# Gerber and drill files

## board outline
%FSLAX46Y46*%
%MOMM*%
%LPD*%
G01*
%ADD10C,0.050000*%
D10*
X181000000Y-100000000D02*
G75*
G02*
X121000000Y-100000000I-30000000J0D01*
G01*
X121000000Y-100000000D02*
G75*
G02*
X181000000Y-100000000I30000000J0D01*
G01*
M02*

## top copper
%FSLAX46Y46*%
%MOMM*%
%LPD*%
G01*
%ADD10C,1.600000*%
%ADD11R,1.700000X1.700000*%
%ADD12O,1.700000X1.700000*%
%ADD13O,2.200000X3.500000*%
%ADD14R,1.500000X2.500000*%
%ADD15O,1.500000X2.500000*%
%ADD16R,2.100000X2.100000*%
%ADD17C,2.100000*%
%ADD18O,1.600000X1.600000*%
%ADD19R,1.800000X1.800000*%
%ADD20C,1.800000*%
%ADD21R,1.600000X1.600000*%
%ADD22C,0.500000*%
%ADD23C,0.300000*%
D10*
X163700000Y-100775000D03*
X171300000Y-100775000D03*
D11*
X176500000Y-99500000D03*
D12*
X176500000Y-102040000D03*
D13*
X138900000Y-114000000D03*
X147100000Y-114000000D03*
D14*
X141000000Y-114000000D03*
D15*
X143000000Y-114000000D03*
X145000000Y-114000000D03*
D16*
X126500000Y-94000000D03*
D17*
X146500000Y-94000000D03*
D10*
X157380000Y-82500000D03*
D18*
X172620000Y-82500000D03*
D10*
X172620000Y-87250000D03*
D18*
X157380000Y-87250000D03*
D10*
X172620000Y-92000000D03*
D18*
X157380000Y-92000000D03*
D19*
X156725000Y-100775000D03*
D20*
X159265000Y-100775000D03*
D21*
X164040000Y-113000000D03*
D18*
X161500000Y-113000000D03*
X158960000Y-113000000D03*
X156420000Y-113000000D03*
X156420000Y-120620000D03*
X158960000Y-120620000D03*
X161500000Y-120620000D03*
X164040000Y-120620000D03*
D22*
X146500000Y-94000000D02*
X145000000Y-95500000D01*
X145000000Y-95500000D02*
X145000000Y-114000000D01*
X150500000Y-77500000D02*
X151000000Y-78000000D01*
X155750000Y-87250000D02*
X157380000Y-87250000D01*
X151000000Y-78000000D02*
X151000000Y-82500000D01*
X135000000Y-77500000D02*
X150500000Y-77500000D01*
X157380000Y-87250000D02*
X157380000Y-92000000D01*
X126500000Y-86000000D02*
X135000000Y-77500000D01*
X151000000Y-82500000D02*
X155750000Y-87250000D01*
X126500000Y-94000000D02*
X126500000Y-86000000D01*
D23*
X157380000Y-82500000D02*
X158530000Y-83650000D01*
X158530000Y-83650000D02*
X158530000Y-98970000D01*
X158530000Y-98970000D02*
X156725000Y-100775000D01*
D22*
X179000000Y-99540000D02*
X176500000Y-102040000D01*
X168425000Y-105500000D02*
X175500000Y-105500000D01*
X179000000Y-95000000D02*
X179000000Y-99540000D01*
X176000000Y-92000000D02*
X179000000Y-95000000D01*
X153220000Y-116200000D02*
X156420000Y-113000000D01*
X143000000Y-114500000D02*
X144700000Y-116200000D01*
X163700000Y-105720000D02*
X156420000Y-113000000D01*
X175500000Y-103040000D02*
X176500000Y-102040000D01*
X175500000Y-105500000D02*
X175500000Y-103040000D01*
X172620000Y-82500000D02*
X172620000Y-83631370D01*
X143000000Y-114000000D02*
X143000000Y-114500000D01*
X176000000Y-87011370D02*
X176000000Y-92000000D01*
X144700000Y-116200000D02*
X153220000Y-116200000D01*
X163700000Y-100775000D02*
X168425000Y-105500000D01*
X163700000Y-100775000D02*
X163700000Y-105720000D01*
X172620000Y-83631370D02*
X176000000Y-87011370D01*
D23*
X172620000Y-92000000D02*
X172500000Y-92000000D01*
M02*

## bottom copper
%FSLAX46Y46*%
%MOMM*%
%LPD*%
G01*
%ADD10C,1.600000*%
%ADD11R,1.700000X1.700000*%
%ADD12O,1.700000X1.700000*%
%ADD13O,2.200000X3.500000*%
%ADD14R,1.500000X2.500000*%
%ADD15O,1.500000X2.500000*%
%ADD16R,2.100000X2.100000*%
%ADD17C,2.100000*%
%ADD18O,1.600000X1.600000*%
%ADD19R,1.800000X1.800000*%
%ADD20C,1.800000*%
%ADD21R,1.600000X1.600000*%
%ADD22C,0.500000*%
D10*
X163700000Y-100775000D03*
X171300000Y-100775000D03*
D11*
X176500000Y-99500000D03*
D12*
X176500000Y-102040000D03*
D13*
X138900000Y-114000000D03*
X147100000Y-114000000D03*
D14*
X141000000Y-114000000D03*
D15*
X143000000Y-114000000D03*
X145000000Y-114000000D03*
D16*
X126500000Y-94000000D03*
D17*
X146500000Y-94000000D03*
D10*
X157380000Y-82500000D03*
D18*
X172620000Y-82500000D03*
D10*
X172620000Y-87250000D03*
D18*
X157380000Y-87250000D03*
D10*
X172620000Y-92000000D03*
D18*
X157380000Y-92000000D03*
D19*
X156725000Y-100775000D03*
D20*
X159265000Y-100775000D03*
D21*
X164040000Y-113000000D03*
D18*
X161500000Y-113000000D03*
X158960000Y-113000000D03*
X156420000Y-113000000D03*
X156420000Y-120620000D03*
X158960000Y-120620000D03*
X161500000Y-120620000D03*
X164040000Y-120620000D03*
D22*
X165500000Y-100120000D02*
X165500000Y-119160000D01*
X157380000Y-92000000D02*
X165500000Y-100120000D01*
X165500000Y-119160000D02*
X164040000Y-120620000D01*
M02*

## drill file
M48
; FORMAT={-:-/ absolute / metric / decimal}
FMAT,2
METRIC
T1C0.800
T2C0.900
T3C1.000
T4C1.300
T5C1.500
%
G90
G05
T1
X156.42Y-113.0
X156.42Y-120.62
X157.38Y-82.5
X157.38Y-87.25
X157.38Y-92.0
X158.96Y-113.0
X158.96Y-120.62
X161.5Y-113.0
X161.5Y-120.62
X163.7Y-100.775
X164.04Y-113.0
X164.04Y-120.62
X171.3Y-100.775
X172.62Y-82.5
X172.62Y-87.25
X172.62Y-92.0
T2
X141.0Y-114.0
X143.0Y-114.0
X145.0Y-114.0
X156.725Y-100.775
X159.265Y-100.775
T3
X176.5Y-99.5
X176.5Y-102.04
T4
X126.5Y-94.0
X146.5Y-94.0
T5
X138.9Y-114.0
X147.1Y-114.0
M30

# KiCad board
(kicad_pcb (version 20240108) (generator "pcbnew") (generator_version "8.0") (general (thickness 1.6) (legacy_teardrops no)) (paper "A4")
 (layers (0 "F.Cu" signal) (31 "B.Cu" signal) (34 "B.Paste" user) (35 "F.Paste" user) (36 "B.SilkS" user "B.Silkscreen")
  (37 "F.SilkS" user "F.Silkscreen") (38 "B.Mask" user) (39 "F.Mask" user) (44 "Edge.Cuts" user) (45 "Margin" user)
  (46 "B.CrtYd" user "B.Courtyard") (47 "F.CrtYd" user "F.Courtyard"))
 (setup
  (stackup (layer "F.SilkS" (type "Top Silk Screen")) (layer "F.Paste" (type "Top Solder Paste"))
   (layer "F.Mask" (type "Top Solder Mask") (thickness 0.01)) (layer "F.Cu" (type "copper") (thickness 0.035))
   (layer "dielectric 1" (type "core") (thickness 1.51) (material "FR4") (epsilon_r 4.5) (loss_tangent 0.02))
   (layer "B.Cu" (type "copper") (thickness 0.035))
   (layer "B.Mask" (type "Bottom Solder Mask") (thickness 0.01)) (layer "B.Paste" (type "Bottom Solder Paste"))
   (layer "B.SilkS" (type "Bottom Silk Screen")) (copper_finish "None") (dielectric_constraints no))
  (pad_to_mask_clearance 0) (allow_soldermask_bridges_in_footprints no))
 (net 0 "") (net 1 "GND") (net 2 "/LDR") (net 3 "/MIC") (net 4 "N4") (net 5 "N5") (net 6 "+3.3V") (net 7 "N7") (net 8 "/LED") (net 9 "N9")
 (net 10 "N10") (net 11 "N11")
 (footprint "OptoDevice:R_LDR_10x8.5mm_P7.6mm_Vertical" (layer "F.Cu") (at 163.7 100.775)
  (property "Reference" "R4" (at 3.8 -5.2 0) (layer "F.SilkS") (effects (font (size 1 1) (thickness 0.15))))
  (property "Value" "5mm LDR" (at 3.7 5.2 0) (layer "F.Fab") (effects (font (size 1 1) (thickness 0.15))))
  (pad "1" thru_hole circle (at 0 0) (size 1.6 1.6) (drill 0.8) (layers "*.Cu" "*.Mask") (remove_unused_layers no) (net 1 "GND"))
  (pad "2" thru_hole circle (at 7.6 0) (size 1.6 1.6) (drill 0.8) (layers "*.Cu" "*.Mask") (remove_unused_layers no) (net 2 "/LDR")))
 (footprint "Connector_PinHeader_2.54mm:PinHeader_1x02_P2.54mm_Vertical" (layer "F.Cu") (at 176.5 99.5)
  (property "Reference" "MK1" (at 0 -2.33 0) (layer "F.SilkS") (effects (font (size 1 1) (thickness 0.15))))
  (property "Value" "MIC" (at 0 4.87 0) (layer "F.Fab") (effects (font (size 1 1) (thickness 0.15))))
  (pad "1" thru_hole rect (at 0 0) (size 1.7 1.7) (drill 1) (layers "*.Cu" "*.Mask") (remove_unused_layers no) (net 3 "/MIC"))
  (pad "2" thru_hole oval (at 0 2.54) (size 1.7 1.7) (drill 1) (layers "*.Cu" "*.Mask") (remove_unused_layers no) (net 1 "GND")))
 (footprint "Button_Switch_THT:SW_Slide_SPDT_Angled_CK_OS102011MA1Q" (layer "F.Cu") (at 141 114)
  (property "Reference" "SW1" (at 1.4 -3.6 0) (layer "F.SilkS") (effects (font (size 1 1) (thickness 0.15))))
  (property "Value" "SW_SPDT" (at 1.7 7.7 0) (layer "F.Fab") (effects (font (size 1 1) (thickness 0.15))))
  (pad "" thru_hole oval (at -2.1 0) (size 2.2 3.5) (drill 1.5) (layers "*.Cu" "*.Mask") (remove_unused_layers no))
  (pad "" thru_hole oval (at 6.1 0) (size 2.2 3.5) (drill 1.5) (layers "*.Cu" "*.Mask") (remove_unused_layers no))
  (pad "1" thru_hole rect (at 0 0) (size 1.5 2.5) (drill 0.9) (layers "*.Cu" "*.Mask") (remove_unused_layers no) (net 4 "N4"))
  (pad "2" thru_hole oval (at 2 0) (size 1.5 2.5) (drill 0.9) (layers "*.Cu" "*.Mask") (remove_unused_layers no) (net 1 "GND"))
  (pad "3" thru_hole oval (at 4 0) (size 1.5 2.5) (drill 0.9) (layers "*.Cu" "*.Mask") (remove_unused_layers no) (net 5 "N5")))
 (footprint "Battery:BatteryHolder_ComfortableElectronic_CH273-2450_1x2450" (layer "F.Cu") (at 126.5 94)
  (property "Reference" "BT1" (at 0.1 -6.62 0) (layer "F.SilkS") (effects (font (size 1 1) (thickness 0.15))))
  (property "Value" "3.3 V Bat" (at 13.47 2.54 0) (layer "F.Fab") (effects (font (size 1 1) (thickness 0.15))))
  (pad "1" thru_hole rect (at 0 0 270) (size 2.1 2.1) (drill 1.3) (layers "*.Cu" "*.Mask") (remove_unused_layers no) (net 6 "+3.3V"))
  (pad "2" thru_hole circle (at 20 0 270) (size 2.1 2.1) (drill 1.3) (layers "*.Cu" "*.Mask") (remove_unused_layers no) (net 5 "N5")))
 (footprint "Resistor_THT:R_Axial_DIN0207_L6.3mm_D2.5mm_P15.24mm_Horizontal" (layer "F.Cu") (at 157.38 82.5)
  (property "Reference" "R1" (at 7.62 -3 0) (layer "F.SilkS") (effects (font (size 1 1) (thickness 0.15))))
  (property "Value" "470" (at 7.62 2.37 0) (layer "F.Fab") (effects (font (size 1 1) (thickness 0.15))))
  (pad "1" thru_hole circle (at 0 0) (size 1.6 1.6) (drill 0.8) (layers "*.Cu" "*.Mask") (remove_unused_layers no) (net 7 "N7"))
  (pad "2" thru_hole oval (at 15.24 0) (size 1.6 1.6) (drill 0.8) (layers "*.Cu" "*.Mask") (remove_unused_layers no) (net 1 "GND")))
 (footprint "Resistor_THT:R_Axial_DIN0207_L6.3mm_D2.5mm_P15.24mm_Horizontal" (layer "F.Cu") (at 172.62 87.25 180)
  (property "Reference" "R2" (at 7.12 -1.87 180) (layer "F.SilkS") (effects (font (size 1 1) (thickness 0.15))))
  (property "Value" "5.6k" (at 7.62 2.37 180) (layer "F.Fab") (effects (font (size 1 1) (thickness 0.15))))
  (pad "1" thru_hole circle (at 0 0 180) (size 1.6 1.6) (drill 0.8) (layers "*.Cu" "*.Mask") (remove_unused_layers no) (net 3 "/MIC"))
  (pad "2" thru_hole oval (at 15.24 0 180) (size 1.6 1.6) (drill 0.8) (layers "*.Cu" "*.Mask") (remove_unused_layers no) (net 6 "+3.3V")))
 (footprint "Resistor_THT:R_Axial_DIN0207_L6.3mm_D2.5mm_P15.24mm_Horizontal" (layer "F.Cu") (at 172.62 92 180)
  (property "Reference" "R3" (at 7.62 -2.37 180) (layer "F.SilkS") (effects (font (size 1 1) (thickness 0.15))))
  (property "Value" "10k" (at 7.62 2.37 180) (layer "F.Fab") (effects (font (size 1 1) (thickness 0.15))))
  (pad "1" thru_hole circle (at 0 0 180) (size 1.6 1.6) (drill 0.8) (layers "*.Cu" "*.Mask") (remove_unused_layers no) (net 2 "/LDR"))
  (pad "2" thru_hole oval (at 15.24 0 180) (size 1.6 1.6) (drill 0.8) (layers "*.Cu" "*.Mask") (remove_unused_layers no) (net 6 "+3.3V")))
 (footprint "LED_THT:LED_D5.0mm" (layer "F.Cu") (at 156.725 100.775)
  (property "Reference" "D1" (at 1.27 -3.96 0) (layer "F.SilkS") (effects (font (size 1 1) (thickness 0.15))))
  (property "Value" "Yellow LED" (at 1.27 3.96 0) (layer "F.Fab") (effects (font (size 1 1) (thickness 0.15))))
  (pad "1" thru_hole rect (at 0 0) (size 1.8 1.8) (drill 0.9) (layers "*.Cu" "*.Mask") (remove_unused_layers no) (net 7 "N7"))
  (pad "2" thru_hole circle (at 2.54 0) (size 1.8 1.8) (drill 0.9) (layers "*.Cu" "*.Mask") (remove_unused_layers no) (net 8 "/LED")))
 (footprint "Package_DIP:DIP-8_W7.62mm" (layer "F.Cu") (at 164.04 113 -90)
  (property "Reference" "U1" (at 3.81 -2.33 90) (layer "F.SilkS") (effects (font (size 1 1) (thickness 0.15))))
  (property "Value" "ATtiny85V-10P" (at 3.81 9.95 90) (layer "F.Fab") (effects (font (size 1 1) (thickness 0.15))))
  (pad "1" thru_hole rect (at 0 0 270) (size 1.6 1.6) (drill 0.8) (layers "*.Cu" "*.Mask") (remove_unused_layers no) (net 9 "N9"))
  (pad "2" thru_hole oval (at 0 2.54 270) (size 1.6 1.6) (drill 0.8) (layers "*.Cu" "*.Mask") (remove_unused_layers no) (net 3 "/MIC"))
  (pad "3" thru_hole oval (at 0 5.08 270) (size 1.6 1.6) (drill 0.8) (layers "*.Cu" "*.Mask") (remove_unused_layers no) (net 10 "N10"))
  (pad "4" thru_hole oval (at 0 7.62 270) (size 1.6 1.6) (drill 0.8) (layers "*.Cu" "*.Mask") (remove_unused_layers no) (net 1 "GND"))
  (pad "5" thru_hole oval (at 7.62 7.62 270) (size 1.6 1.6) (drill 0.8) (layers "*.Cu" "*.Mask") (remove_unused_layers no) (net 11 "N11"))
  (pad "6" thru_hole oval (at 7.62 5.08 270) (size 1.6 1.6) (drill 0.8) (layers "*.Cu" "*.Mask") (remove_unused_layers no) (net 8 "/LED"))
  (pad "7" thru_hole oval (at 7.62 2.54 270) (size 1.6 1.6) (drill 0.8) (layers "*.Cu" "*.Mask") (remove_unused_layers no) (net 2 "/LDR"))
  (pad "8" thru_hole oval (at 7.62 0 270) (size 1.6 1.6) (drill 0.8) (layers "*.Cu" "*.Mask") (remove_unused_layers no) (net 6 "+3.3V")))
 (gr_circle (center 151 100) (end 181 100) (stroke (width 0.05) (type default)) (fill none) (layer "Edge.Cuts"))
 (segment (start 146.5 94) (end 145 95.5) (width 0.5) (layer "F.Cu") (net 5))
 (segment (start 145 95.5) (end 145 114) (width 0.5) (layer "F.Cu") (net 5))
 (segment (start 150.5 77.5) (end 151 78) (width 0.5) (layer "F.Cu") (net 6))
 (segment (start 155.75 87.25) (end 157.38 87.25) (width 0.5) (layer "F.Cu") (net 6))
 (segment (start 151 78) (end 151 82.5) (width 0.5) (layer "F.Cu") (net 6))
 (segment (start 135 77.5) (end 150.5 77.5) (width 0.5) (layer "F.Cu") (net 6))
 (segment (start 157.38 87.25) (end 157.38 92) (width 0.5) (layer "F.Cu") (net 6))
 (segment (start 126.5 86) (end 135 77.5) (width 0.5) (layer "F.Cu") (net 6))
 (segment (start 151 82.5) (end 155.75 87.25) (width 0.5) (layer "F.Cu") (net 6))
 (segment (start 126.5 94) (end 126.5 86) (width 0.5) (layer "F.Cu") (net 6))
 (segment (start 165.5 100.12) (end 165.5 119.16) (width 0.5) (layer "B.Cu") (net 6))
 (segment (start 157.38 92) (end 165.5 100.12) (width 0.5) (layer "B.Cu") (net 6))
 (segment (start 165.5 119.16) (end 164.04 120.62) (width 0.5) (layer "B.Cu") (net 6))
 (segment (start 157.38 82.5) (end 158.53 83.65) (width 0.3) (layer "F.Cu") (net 7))
 (segment (start 158.53 83.65) (end 158.53 98.97) (width 0.3) (layer "F.Cu") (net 7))
 (segment (start 158.53 98.97) (end 156.725 100.775) (width 0.3) (layer "F.Cu") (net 7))
 (segment (start 179 99.54) (end 176.5 102.04) (width 0.5) (layer "F.Cu") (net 1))
 (segment (start 168.425 105.5) (end 175.5 105.5) (width 0.5) (layer "F.Cu") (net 1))
 (segment (start 179 95) (end 179 99.54) (width 0.5) (layer "F.Cu") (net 1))
 (segment (start 176 92) (end 179 95) (width 0.5) (layer "F.Cu") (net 1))
 (segment (start 153.22 116.2) (end 156.42 113) (width 0.5) (layer "F.Cu") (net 1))
 (segment (start 143 114.5) (end 144.7 116.2) (width 0.5) (layer "F.Cu") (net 1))
 (segment (start 163.7 105.72) (end 156.42 113) (width 0.5) (layer "F.Cu") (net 1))
 (segment (start 175.5 103.04) (end 176.5 102.04) (width 0.5) (layer "F.Cu") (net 1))
 (segment (start 175.5 105.5) (end 175.5 103.04) (width 0.5) (layer "F.Cu") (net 1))
 (segment (start 172.62 82.5) (end 172.62 83.63137) (width 0.5) (layer "F.Cu") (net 1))
 (segment (start 143 114) (end 143 114.5) (width 0.5) (layer "F.Cu") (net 1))
 (segment (start 176 87.01137) (end 176 92) (width 0.5) (layer "F.Cu") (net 1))
 (segment (start 144.7 116.2) (end 153.22 116.2) (width 0.5) (layer "F.Cu") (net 1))
 (segment (start 163.7 100.775) (end 168.425 105.5) (width 0.5) (layer "F.Cu") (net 1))
 (segment (start 163.7 100.775) (end 163.7 105.72) (width 0.5) (layer "F.Cu") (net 1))
 (segment (start 172.62 83.63137) (end 176 87.01137) (width 0.5) (layer "F.Cu") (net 1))
 (segment (start 172.62 92) (end 172.5 92) (width 0.3) (layer "F.Cu") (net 2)))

